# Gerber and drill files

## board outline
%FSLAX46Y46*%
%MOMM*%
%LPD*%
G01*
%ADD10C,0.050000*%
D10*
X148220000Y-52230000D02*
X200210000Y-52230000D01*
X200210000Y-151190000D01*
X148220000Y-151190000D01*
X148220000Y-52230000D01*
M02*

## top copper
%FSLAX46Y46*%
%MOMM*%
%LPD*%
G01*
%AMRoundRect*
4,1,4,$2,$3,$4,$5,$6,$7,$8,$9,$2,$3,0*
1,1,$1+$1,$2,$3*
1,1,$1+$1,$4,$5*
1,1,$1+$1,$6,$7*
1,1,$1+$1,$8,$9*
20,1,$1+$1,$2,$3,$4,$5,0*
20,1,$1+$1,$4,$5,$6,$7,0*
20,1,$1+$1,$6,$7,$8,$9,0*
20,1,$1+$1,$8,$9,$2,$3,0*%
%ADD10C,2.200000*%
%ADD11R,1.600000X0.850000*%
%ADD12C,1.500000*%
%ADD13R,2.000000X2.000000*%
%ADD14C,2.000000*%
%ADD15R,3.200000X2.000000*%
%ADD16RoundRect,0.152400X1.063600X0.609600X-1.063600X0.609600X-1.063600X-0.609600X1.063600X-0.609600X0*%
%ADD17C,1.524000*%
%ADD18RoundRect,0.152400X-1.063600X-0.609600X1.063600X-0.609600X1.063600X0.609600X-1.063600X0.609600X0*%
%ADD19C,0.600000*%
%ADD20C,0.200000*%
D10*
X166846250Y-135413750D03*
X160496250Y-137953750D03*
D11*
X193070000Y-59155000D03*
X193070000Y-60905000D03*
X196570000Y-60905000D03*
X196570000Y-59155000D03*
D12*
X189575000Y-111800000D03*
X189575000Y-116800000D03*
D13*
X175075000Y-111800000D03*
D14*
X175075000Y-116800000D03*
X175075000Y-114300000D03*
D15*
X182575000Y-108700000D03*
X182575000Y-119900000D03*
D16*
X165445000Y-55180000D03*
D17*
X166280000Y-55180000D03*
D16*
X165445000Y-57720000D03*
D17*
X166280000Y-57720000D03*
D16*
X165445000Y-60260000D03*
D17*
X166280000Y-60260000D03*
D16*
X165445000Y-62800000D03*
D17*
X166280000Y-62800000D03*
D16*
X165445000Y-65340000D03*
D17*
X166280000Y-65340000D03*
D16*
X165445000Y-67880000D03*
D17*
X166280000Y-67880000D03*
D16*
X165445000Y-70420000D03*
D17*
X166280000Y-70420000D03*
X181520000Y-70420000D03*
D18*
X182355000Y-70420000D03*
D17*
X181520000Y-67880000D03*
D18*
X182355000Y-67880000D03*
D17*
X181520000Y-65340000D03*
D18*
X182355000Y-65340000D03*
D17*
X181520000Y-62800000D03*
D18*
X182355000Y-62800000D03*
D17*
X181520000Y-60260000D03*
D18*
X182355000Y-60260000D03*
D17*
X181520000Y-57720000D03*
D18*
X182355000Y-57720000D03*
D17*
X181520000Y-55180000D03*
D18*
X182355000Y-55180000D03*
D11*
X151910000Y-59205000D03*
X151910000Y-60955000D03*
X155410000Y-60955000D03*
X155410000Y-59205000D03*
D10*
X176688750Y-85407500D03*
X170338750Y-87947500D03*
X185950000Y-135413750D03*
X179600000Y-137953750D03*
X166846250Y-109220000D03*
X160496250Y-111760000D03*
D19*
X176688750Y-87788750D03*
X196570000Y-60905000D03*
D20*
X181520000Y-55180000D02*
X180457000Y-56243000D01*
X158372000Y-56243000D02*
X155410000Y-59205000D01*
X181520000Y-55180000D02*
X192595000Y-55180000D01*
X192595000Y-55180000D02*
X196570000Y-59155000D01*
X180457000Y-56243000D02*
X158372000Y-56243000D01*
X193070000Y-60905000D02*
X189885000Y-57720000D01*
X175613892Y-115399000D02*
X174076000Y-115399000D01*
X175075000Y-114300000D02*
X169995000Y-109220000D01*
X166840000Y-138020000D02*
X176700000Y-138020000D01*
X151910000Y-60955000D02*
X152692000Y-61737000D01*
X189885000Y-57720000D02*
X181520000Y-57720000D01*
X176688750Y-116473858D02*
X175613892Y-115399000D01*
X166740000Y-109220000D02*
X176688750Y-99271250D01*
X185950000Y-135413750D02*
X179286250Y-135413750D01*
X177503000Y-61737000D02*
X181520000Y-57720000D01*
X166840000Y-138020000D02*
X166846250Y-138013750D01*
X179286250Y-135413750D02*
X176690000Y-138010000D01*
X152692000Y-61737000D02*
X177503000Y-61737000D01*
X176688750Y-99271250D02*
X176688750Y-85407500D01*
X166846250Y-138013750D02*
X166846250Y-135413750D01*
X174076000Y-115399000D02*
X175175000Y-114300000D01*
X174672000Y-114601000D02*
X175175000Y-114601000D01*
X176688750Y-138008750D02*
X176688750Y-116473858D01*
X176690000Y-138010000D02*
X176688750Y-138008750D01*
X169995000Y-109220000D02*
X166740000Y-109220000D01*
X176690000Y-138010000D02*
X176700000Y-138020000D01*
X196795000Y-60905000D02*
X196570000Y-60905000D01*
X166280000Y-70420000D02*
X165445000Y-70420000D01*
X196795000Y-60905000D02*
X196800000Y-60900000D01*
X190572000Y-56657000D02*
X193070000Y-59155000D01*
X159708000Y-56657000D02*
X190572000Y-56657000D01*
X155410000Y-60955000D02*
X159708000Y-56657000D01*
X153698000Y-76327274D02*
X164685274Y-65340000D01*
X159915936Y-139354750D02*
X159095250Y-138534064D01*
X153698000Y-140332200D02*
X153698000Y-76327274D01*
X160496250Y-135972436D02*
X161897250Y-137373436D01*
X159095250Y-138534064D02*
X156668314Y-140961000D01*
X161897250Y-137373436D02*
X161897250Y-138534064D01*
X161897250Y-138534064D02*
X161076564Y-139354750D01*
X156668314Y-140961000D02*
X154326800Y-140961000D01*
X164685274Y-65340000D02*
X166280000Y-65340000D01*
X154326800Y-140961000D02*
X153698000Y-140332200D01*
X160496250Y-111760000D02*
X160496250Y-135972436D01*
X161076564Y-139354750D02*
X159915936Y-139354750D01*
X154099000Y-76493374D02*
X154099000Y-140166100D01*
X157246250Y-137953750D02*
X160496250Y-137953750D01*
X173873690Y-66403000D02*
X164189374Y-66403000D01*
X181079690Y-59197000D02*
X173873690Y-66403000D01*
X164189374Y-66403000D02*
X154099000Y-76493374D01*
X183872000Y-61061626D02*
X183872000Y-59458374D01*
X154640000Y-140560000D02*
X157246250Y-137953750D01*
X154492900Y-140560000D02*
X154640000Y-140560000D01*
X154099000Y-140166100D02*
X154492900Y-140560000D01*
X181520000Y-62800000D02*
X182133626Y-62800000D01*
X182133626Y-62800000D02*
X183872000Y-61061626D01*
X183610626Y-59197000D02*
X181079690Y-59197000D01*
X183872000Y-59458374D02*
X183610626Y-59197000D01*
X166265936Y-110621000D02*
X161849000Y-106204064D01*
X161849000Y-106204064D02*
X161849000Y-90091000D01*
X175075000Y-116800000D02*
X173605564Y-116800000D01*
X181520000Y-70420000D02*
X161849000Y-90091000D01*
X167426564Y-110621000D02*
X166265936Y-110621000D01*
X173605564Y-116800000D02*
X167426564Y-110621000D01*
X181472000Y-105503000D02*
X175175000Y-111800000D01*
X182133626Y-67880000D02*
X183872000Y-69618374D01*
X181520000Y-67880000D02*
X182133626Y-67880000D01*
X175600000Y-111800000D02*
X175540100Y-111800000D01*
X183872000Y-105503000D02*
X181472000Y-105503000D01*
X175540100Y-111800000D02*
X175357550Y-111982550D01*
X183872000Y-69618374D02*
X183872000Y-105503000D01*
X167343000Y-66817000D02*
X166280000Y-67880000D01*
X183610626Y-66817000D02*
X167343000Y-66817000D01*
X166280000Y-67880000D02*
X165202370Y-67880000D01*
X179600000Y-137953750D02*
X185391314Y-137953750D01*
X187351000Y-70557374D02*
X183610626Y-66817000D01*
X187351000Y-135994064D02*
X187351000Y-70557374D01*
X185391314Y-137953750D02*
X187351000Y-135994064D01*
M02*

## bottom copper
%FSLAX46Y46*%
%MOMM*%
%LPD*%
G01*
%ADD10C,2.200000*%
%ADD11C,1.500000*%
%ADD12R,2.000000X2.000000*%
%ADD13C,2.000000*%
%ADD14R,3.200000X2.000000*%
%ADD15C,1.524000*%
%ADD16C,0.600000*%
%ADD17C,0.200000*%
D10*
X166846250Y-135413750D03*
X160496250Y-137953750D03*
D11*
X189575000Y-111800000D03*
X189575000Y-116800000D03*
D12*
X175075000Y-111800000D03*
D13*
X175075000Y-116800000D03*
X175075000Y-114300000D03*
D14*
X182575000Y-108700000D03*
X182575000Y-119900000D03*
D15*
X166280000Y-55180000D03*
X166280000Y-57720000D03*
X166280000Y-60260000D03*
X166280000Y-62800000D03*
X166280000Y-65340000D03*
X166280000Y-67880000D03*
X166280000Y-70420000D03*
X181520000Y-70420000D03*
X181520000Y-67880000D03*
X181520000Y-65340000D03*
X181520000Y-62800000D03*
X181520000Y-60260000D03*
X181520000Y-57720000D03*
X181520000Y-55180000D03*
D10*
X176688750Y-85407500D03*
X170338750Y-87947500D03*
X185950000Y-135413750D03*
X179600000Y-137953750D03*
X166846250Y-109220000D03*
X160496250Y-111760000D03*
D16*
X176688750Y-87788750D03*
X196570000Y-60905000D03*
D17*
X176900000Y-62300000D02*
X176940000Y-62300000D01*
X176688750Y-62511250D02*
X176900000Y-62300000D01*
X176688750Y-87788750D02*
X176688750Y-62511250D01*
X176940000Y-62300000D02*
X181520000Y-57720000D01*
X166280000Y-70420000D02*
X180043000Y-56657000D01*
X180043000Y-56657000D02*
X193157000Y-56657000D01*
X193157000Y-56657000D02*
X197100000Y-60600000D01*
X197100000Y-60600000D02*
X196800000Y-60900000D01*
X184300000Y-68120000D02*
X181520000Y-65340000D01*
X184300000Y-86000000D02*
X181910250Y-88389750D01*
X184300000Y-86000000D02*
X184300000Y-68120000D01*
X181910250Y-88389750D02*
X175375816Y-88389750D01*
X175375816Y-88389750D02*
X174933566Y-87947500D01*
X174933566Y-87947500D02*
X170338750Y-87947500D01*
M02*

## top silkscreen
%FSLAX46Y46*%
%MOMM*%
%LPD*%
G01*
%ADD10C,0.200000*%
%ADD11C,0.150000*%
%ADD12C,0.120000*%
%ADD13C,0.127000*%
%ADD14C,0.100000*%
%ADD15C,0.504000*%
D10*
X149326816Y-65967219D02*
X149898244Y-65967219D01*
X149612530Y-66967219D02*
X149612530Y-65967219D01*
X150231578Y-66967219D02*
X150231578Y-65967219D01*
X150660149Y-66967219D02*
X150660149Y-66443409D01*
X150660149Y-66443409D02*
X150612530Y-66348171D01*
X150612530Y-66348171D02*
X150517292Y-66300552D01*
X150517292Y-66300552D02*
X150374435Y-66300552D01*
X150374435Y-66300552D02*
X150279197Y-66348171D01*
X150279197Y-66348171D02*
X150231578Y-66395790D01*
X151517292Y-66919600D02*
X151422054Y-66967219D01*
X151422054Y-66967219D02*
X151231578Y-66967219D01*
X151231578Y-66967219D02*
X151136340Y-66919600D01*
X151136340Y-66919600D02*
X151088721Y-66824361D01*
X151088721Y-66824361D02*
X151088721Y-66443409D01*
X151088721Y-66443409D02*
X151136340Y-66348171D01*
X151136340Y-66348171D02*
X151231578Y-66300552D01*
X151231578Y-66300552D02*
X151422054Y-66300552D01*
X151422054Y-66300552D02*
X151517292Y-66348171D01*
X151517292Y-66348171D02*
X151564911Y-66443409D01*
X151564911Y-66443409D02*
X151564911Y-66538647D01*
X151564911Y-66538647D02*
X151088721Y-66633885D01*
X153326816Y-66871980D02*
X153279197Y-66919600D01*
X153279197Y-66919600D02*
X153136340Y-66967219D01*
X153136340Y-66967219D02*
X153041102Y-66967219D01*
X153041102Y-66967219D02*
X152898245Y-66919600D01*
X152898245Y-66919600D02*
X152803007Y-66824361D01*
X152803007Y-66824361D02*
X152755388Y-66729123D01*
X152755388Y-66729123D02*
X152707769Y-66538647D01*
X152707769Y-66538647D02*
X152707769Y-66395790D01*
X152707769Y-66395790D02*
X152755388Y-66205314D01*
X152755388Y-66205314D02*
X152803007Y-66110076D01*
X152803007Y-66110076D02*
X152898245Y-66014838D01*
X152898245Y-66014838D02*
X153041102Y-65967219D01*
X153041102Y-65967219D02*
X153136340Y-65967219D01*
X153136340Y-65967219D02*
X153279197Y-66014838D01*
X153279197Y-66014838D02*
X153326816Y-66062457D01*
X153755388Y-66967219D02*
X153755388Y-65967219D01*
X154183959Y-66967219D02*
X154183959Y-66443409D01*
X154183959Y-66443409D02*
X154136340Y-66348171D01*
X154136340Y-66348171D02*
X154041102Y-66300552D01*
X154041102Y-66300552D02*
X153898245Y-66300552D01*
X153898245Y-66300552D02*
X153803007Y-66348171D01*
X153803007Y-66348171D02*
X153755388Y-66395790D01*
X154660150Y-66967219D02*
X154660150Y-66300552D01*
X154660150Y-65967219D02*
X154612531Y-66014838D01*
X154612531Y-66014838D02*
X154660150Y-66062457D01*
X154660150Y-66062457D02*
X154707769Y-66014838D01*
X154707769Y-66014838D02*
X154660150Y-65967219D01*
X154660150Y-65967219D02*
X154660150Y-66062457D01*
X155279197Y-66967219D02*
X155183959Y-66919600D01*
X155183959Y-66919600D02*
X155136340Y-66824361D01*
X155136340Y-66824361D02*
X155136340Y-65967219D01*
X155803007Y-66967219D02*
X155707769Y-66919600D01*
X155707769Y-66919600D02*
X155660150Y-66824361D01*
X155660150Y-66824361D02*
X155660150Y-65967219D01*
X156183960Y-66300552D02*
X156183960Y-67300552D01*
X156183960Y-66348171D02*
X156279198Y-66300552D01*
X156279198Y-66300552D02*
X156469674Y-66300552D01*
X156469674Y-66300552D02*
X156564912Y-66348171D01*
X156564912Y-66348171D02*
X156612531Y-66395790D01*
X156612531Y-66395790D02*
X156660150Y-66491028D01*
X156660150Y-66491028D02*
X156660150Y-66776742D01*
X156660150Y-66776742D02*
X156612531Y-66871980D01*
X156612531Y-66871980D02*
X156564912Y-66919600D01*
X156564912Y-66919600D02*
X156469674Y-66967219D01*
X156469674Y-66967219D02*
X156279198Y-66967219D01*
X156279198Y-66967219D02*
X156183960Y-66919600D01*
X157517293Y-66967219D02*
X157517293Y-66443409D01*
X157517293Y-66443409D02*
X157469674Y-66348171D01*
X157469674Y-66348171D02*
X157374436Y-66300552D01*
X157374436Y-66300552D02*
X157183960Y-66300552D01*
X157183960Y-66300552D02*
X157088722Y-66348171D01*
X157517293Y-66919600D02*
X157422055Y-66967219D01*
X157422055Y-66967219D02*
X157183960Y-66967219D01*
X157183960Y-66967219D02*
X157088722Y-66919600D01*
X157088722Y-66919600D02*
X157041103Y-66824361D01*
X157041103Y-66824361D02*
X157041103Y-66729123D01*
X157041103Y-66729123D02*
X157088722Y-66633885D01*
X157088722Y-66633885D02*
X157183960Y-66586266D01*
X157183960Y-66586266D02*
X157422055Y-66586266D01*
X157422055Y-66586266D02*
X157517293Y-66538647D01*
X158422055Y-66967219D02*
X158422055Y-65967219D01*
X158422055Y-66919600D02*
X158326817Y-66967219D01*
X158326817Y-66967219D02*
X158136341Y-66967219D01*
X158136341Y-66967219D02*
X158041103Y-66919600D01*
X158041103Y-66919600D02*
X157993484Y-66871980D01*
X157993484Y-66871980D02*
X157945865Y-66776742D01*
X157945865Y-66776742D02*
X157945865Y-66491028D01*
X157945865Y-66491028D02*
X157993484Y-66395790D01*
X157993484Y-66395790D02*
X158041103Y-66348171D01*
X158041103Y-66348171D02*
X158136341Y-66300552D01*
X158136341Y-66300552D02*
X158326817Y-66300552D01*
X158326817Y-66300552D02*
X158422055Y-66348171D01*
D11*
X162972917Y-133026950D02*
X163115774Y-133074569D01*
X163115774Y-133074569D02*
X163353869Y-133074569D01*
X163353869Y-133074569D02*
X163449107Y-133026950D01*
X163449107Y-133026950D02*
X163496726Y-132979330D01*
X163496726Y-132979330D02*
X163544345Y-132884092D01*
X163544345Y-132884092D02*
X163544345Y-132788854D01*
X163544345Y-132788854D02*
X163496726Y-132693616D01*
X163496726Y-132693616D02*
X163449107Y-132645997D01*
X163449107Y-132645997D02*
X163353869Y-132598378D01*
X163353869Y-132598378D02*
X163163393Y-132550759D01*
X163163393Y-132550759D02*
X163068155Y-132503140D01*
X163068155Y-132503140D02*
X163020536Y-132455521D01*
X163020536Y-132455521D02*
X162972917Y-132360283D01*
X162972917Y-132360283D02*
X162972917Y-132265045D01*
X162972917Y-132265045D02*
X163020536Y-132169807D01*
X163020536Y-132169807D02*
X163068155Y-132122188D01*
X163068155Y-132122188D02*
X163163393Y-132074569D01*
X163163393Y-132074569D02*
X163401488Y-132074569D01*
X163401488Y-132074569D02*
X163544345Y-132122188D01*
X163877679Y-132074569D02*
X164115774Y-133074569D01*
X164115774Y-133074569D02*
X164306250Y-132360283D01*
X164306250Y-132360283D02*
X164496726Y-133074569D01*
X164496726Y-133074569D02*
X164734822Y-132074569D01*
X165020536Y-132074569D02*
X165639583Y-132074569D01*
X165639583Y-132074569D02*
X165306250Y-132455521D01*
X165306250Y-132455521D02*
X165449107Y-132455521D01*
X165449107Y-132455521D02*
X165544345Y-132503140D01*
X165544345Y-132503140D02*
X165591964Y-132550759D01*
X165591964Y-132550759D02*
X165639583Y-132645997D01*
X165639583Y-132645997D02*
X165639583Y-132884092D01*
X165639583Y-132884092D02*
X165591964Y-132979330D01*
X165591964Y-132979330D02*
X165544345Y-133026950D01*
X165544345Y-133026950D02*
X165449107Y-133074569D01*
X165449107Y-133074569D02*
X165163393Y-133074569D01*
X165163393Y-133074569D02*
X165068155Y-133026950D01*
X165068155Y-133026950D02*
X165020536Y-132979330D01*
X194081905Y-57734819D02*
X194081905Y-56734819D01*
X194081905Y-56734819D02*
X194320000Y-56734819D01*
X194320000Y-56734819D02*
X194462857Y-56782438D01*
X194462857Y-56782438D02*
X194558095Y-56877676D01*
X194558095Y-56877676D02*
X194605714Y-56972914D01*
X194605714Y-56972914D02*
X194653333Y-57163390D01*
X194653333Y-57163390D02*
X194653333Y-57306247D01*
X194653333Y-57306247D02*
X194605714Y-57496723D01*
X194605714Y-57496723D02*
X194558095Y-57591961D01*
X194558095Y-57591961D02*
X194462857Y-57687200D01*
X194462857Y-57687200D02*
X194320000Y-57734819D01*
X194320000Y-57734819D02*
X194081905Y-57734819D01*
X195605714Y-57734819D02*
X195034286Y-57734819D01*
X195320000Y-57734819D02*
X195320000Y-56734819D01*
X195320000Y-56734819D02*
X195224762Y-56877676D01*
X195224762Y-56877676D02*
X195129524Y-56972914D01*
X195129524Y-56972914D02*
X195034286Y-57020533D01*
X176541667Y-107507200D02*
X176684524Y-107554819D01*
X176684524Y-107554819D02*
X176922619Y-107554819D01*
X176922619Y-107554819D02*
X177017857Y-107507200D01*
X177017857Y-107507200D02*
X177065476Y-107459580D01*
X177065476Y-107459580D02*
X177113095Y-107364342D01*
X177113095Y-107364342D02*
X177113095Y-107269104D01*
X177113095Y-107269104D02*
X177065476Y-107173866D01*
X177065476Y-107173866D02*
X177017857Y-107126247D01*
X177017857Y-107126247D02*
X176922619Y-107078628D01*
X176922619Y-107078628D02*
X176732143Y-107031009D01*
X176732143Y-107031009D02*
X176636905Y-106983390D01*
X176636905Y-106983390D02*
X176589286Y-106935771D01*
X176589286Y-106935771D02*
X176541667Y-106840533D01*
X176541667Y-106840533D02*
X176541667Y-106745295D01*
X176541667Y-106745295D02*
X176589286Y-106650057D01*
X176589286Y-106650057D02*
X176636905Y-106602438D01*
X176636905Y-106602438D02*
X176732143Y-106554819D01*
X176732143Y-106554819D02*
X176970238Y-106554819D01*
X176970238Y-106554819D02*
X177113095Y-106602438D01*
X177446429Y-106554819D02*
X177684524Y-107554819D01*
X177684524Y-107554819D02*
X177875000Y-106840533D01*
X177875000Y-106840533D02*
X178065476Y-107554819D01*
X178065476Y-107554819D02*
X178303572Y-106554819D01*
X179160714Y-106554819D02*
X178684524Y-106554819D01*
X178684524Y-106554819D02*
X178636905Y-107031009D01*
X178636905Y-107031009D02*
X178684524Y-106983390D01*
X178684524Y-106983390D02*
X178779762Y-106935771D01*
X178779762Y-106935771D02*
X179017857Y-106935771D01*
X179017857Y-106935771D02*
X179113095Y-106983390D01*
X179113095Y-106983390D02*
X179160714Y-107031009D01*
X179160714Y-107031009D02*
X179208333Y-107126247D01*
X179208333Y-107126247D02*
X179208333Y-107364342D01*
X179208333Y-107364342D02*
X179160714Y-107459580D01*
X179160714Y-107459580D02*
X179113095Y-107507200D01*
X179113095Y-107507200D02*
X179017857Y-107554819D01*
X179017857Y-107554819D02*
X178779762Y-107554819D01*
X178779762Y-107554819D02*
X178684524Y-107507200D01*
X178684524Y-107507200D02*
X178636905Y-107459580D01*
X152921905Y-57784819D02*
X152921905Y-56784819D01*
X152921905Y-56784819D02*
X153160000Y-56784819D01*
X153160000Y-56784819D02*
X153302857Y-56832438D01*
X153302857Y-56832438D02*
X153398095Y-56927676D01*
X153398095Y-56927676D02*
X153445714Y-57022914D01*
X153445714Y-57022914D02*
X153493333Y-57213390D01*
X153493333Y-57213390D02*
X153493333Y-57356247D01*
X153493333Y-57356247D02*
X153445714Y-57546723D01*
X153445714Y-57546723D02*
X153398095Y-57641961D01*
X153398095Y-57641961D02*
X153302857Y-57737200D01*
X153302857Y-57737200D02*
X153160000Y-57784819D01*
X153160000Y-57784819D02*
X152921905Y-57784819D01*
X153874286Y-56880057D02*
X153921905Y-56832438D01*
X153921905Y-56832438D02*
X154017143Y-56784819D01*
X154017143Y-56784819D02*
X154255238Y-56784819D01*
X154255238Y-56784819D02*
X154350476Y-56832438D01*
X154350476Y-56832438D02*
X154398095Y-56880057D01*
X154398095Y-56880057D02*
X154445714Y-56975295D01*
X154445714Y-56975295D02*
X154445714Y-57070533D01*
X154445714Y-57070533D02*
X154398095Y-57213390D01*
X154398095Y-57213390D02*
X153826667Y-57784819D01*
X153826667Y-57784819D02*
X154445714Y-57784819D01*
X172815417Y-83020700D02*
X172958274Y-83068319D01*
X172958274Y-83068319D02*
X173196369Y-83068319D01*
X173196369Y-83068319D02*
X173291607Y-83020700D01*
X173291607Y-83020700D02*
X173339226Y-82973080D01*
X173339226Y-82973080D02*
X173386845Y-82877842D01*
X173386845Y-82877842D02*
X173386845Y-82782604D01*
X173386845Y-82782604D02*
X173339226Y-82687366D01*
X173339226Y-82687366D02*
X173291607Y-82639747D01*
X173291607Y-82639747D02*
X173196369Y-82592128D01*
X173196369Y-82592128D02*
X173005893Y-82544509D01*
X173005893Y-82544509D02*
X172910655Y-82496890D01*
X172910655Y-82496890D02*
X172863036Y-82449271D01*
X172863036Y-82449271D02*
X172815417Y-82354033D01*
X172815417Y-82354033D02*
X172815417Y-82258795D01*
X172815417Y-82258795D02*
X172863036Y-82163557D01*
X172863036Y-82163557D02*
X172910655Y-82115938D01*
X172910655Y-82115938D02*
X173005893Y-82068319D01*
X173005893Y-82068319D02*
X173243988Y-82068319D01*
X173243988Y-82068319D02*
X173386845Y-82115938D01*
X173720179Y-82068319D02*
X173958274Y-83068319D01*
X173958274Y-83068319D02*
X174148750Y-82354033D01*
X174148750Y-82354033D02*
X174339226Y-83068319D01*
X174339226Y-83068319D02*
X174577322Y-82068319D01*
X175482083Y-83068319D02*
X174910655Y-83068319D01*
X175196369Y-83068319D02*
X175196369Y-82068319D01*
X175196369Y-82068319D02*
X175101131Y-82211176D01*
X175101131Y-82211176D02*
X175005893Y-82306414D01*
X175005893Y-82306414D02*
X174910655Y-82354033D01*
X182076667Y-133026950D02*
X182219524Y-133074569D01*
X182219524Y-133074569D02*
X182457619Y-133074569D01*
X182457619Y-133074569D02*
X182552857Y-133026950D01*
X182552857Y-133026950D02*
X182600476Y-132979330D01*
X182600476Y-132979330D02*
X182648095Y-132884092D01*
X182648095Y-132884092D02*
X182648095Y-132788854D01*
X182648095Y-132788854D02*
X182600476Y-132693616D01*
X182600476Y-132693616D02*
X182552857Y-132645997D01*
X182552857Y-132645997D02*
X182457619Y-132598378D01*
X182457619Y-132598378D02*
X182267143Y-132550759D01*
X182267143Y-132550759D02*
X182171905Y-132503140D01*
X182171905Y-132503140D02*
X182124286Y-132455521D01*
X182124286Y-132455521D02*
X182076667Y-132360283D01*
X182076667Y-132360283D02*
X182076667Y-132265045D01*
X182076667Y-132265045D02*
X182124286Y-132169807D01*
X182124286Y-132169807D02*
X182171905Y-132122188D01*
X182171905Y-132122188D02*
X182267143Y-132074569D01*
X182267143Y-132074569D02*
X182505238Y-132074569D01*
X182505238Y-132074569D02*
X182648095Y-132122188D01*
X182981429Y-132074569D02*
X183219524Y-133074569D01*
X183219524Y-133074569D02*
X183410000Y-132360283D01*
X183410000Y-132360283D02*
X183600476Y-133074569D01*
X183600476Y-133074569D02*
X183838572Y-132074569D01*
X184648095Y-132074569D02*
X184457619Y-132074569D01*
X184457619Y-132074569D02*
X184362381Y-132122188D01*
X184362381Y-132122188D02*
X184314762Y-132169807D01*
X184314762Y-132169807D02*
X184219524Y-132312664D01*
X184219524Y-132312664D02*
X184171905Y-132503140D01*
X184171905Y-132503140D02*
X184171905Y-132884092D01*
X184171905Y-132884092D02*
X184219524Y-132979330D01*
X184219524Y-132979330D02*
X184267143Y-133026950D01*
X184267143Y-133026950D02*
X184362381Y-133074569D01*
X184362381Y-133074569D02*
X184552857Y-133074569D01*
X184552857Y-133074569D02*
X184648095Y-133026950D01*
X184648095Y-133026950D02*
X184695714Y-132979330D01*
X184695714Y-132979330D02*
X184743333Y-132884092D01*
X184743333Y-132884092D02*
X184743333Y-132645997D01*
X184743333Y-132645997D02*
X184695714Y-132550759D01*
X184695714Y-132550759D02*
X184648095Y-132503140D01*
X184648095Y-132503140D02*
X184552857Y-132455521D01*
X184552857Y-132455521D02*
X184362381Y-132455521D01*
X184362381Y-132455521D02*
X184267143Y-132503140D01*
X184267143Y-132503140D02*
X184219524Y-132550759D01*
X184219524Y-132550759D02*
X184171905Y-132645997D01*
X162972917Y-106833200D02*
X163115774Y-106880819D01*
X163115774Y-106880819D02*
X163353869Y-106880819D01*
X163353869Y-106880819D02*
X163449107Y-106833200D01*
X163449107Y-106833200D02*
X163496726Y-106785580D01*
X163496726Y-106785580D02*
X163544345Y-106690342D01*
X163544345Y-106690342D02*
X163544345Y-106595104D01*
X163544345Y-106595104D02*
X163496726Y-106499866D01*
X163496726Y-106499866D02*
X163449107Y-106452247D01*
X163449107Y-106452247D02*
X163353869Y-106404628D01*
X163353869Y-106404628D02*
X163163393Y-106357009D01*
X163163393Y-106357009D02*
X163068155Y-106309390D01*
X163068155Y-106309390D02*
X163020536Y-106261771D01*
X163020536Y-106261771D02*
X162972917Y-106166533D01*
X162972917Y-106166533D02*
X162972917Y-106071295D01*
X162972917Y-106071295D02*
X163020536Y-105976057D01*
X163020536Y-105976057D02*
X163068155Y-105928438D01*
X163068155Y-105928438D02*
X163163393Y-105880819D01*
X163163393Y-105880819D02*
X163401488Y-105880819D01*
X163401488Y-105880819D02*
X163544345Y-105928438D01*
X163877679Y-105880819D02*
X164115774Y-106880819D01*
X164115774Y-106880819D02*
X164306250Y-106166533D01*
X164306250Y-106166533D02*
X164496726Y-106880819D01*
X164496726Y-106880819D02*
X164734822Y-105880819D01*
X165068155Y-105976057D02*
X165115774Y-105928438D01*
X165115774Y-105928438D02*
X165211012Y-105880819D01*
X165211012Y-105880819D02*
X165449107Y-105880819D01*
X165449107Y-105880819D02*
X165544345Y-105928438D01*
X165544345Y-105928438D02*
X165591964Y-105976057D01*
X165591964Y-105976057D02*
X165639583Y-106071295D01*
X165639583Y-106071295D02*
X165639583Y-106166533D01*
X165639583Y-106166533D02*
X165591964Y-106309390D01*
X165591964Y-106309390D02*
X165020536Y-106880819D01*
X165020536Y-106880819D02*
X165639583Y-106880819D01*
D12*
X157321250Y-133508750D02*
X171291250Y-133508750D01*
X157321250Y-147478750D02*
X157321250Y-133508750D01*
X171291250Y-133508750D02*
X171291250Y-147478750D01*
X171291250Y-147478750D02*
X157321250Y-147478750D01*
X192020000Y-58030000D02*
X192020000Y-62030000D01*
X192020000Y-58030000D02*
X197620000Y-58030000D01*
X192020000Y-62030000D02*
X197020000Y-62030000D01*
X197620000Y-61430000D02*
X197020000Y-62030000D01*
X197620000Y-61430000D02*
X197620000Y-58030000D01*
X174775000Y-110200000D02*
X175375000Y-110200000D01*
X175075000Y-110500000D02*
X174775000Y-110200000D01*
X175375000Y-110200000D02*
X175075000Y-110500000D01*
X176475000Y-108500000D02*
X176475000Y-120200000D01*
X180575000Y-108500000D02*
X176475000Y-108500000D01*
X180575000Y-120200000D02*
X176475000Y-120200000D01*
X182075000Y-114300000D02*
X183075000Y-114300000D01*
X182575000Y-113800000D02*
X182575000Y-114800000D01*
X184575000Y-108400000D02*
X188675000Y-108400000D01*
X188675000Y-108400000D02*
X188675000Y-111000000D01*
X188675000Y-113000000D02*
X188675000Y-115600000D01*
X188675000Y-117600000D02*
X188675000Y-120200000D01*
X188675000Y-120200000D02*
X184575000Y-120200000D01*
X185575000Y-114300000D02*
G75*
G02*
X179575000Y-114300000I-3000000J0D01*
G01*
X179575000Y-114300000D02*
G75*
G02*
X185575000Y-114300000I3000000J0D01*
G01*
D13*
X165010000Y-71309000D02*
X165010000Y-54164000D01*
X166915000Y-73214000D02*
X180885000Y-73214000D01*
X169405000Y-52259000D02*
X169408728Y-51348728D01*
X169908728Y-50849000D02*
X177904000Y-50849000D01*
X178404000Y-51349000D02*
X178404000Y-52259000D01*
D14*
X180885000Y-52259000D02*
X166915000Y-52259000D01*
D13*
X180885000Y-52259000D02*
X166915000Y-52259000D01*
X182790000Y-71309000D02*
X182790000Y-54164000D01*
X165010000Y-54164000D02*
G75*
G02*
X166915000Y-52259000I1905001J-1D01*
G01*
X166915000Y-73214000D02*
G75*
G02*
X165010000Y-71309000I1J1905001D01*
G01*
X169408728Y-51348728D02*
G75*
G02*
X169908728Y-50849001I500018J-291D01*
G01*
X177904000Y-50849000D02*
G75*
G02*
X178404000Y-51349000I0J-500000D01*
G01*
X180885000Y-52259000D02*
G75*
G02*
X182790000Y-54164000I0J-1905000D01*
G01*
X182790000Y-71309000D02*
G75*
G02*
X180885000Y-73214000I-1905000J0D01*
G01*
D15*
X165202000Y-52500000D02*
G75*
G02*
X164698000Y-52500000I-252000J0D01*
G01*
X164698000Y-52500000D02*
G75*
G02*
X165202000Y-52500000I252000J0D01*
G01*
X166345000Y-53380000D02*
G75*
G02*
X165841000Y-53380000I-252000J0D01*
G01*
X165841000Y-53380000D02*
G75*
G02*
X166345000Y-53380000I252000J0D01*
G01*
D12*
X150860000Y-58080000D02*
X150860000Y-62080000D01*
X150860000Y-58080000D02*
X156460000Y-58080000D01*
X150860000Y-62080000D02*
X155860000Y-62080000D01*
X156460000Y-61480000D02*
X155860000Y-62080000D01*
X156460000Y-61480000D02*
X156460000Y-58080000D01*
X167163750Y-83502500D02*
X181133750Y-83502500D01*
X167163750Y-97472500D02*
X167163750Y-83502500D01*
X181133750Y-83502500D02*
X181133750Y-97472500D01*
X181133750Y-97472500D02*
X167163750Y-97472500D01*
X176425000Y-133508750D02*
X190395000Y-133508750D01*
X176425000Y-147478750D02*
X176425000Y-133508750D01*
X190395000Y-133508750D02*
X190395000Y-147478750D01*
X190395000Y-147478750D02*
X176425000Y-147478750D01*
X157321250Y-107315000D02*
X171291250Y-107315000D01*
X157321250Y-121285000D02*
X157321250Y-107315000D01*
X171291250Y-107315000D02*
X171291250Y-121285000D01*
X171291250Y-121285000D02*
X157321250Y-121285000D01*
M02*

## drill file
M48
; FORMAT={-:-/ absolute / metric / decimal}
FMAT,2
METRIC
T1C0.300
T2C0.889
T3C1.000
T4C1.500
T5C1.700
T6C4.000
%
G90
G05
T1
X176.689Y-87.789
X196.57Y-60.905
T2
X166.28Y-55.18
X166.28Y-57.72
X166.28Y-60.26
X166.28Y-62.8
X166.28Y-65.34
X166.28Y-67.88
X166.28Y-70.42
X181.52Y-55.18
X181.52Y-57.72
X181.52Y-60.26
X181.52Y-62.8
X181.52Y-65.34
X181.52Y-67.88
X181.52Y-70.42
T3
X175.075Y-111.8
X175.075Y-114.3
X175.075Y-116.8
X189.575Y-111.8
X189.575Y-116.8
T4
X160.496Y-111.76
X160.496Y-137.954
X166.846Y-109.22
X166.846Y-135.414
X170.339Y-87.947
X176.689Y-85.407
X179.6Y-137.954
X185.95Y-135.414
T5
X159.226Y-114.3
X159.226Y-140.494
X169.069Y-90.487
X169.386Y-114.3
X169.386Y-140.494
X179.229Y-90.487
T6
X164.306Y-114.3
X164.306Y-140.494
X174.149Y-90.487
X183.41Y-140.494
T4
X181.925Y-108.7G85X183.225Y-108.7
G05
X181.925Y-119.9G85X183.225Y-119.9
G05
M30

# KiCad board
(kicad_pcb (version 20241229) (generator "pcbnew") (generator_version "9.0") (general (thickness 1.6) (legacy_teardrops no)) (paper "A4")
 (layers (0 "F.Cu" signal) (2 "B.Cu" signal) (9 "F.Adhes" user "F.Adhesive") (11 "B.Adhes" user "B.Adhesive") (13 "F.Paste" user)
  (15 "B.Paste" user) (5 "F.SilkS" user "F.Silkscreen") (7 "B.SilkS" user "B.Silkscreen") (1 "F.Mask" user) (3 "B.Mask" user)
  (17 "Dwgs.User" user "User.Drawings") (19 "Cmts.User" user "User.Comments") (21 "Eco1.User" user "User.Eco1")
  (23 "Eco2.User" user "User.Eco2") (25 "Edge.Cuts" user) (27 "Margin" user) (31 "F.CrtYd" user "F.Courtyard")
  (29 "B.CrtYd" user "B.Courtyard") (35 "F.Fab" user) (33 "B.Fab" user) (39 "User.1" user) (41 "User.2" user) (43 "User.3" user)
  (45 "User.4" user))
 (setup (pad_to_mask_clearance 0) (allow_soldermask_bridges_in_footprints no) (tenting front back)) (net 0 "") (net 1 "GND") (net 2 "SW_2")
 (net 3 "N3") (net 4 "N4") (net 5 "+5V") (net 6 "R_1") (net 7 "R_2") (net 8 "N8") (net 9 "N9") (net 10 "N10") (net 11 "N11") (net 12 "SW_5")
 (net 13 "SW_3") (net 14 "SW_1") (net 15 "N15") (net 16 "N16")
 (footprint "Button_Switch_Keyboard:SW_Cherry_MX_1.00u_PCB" (layer "F.Cu") (at 166.84625 135.41375)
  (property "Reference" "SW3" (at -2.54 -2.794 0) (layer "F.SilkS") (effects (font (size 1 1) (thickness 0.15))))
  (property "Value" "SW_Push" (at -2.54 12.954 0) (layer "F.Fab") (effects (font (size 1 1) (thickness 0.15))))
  (fp_line (start -9.525 -1.905) (end 4.445 -1.905) (stroke (width 0.12) (type solid)) (layer "F.SilkS"))
  (fp_line (start -9.525 12.065) (end -9.525 -1.905) (stroke (width 0.12) (type solid)) (layer "F.SilkS"))
  (fp_line (start 4.445 -1.905) (end 4.445 12.065) (stroke (width 0.12) (type solid)) (layer "F.SilkS"))
  (fp_line (start 4.445 12.065) (end -9.525 12.065) (stroke (width 0.12) (type solid)) (layer "F.SilkS"))
  (pad "" np_thru_hole circle (at -7.62 5.08) (size 1.7 1.7) (drill 1.7) (layers "*.Cu" "*.Mask"))
  (pad "" np_thru_hole circle (at -2.54 5.08) (size 4 4) (drill 4) (layers "*.Cu" "*.Mask"))
  (pad "" np_thru_hole circle (at 2.54 5.08) (size 1.7 1.7) (drill 1.7) (layers "*.Cu" "*.Mask"))
  (pad "1" thru_hole circle (at 0 0) (size 2.2 2.2) (drill 1.5) (layers "*.Cu" "*.Mask") (remove_unused_layers no) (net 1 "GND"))
  (pad "2" thru_hole circle (at -6.35 2.54) (size 2.2 2.2) (drill 1.5) (layers "*.Cu" "*.Mask") (remove_unused_layers no) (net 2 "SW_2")))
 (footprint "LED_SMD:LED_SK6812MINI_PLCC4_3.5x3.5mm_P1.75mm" (layer "F.Cu") (at 194.82 60.03)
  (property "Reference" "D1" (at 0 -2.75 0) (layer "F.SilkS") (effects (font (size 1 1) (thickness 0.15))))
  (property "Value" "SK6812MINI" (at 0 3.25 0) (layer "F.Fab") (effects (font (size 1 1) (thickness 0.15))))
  (fp_line (start -2.8 -2) (end -2.8 2) (stroke (width 0.12) (type default)) (layer "F.SilkS"))
  (fp_line (start -2.8 -2) (end 2.8 -2) (stroke (width 0.12) (type solid)) (layer "F.SilkS"))
  (fp_line (start -2.8 2) (end 2.2 2) (stroke (width 0.12) (type solid)) (layer "F.SilkS"))
  (fp_line (start 2.8 1.4) (end 2.2 2) (stroke (width 0.12) (type default)) (layer "F.SilkS"))
  (fp_line (start 2.8 1.4) (end 2.8 -2) (stroke (width 0.12) (type solid)) (layer "F.SilkS"))
  (pad "1" smd rect (at -1.75 -0.875) (size 1.6 0.85) (layers "F.Cu" "F.Mask" "F.Paste") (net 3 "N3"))
  (pad "2" smd rect (at -1.75 0.875) (size 1.6 0.85) (layers "F.Cu" "F.Mask" "F.Paste") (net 1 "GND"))
  (pad "3" smd rect (at 1.75 0.875) (size 1.6 0.85) (layers "F.Cu" "F.Mask" "F.Paste") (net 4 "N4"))
  (pad "4" smd rect (at 1.75 -0.875) (size 1.6 0.85) (layers "F.Cu" "F.Mask" "F.Paste") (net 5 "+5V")))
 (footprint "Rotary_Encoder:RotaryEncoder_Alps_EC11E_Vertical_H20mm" (layer "F.Cu") (at 175.075 111.8)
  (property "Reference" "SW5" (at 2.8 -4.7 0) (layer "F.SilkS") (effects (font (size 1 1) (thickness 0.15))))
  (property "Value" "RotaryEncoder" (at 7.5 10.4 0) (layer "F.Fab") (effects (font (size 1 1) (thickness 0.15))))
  (fp_line (start -0.3 -1.6) (end 0.3 -1.6) (stroke (width 0.12) (type solid)) (layer "F.SilkS"))
  (fp_line (start 0 -1.3) (end -0.3 -1.6) (stroke (width 0.12) (type solid)) (layer "F.SilkS"))
  (fp_line (start 0.3 -1.6) (end 0 -1.3) (stroke (width 0.12) (type solid)) (layer "F.SilkS"))
  (fp_line (start 1.4 -3.3) (end 1.4 8.4) (stroke (width 0.12) (type solid)) (layer "F.SilkS"))
  (fp_line (start 5.5 -3.3) (end 1.4 -3.3) (stroke (width 0.12) (type solid)) (layer "F.SilkS"))
  (fp_line (start 5.5 8.4) (end 1.4 8.4) (stroke (width 0.12) (type solid)) (layer "F.SilkS"))
  (fp_line (start 7 2.5) (end 8 2.5) (stroke (width 0.12) (type solid)) (layer "F.SilkS"))
  (fp_line (start 7.5 2) (end 7.5 3) (stroke (width 0.12) (type solid)) (layer "F.SilkS"))
  (fp_line (start 9.5 -3.4) (end 13.6 -3.4) (stroke (width 0.12) (type solid)) (layer "F.SilkS"))
  (fp_line (start 13.6 -3.4) (end 13.6 -0.8) (stroke (width 0.12) (type solid)) (layer "F.SilkS"))
  (fp_line (start 13.6 1.2) (end 13.6 3.8) (stroke (width 0.12) (type solid)) (layer "F.SilkS"))
  (fp_line (start 13.6 5.8) (end 13.6 8.4) (stroke (width 0.12) (type solid)) (layer "F.SilkS"))
  (fp_line (start 13.6 8.4) (end 9.5 8.4) (stroke (width 0.12) (type solid)) (layer "F.SilkS"))
  (fp_circle (center 7.5 2.5) (end 10.5 2.5) (stroke (width 0.12) (type solid)) (fill no) (layer "F.SilkS"))
  (pad "" thru_hole circle (at 14.5 0) (size 1.5 1.5) (drill 1) (layers "*.Cu" "*.Mask") (remove_unused_layers no))
  (pad "" thru_hole circle (at 14.5 5) (size 1.5 1.5) (drill 1) (layers "*.Cu" "*.Mask") (remove_unused_layers no))
  (pad "A" thru_hole rect (at 0 0) (size 2 2) (drill 1) (layers "*.Cu" "*.Mask") (remove_unused_layers no) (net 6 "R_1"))
  (pad "B" thru_hole circle (at 0 5) (size 2 2) (drill 1) (layers "*.Cu" "*.Mask") (remove_unused_layers no) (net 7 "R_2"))
  (pad "C" thru_hole circle (at 0 2.5) (size 2 2) (drill 1) (layers "*.Cu" "*.Mask") (remove_unused_layers no) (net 1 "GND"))
  (pad "MP" thru_hole rect (at 7.5 -3.1) (size 3.2 2) (drill oval 2.8 1.5) (layers "*.Cu" "*.Mask") (remove_unused_layers no))
  (pad "MP" thru_hole rect (at 7.5 8.1) (size 3.2 2) (drill oval 2.8 1.5) (layers "*.Cu" "*.Mask") (remove_unused_layers no)))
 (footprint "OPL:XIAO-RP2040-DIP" (layer "F.Cu") (at 173.9 62.8)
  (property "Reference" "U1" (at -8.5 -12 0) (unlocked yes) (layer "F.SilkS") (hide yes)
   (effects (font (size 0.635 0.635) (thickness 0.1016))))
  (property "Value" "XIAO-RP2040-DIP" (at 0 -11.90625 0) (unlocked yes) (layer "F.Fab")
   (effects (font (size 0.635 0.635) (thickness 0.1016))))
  (fp_line (start -8.89 8.509) (end -8.89 -8.636) (stroke (width 0.127) (type solid)) (layer "F.SilkS"))
  (fp_line (start -6.985 10.414) (end 6.985 10.414) (stroke (width 0.127) (type solid)) (layer "F.SilkS"))
  (fp_line (start -4.495 -10.541) (end -4.491272 -11.451272) (stroke (width 0.127) (type solid)) (layer "F.SilkS"))
  (fp_line (start -3.991272 -11.951) (end 4.004 -11.951) (stroke (width 0.127) (type solid)) (layer "F.SilkS"))
  (fp_line (start 4.504 -11.451) (end 4.504 -10.541) (stroke (width 0.127) (type solid)) (layer "F.SilkS"))
  (fp_line (start 6.985 -10.541) (end -6.985 -10.541) (stroke (width 0.1) (type solid)) (layer "F.SilkS"))
  (fp_line (start 6.985 -10.541) (end -6.985 -10.541) (stroke (width 0.127) (type solid)) (layer "F.SilkS"))
  (fp_line (start 8.89 8.509) (end 8.89 -8.636) (stroke (width 0.127) (type solid)) (layer "F.SilkS"))
  (fp_arc (start -8.89 -8.636) (mid -8.332038 -9.983038) (end -6.985 -10.541) (stroke (width 0.127) (type solid)) (layer "F.SilkS"))
  (fp_arc (start -6.985 10.414) (mid -8.332038 9.856038) (end -8.89 8.509) (stroke (width 0.127) (type solid)) (layer "F.SilkS"))
  (fp_arc (start -4.491272 -11.451272) (mid -4.344728 -11.80464) (end -3.991272 -11.951) (stroke (width 0.127) (type default))
   (layer "F.SilkS"))
  (fp_arc (start 4.004 -11.951) (mid 4.357553 -11.804553) (end 4.504 -11.451) (stroke (width 0.127) (type default)) (layer "F.SilkS"))
  (fp_arc (start 6.985 -10.541) (mid 8.332038 -9.983038) (end 8.89 -8.636) (stroke (width 0.127) (type solid)) (layer "F.SilkS"))
  (fp_arc (start 8.89 8.509) (mid 8.332038 9.856038) (end 6.985 10.414) (stroke (width 0.127) (type solid)) (layer "F.SilkS"))
  (fp_circle (center -8.95 -10.3) (end -8.95 -10.554) (stroke (width 0.5) (type solid)) (fill yes) (layer "F.SilkS"))
  (fp_circle (center -7.807 -9.42) (end -7.807 -9.674) (stroke (width 0.5) (type solid)) (fill yes) (layer "F.SilkS"))
  (pad "1" smd roundrect (at -8.455 -7.62 180) (size 2.432 1.524) (layers "F.Cu" "F.Mask") (roundrect_rratio 0.1) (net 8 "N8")
   (thermal_bridge_angle 45))
  (pad "1" thru_hole circle (at -7.62 -7.62 180) (size 1.524 1.524) (drill 0.889) (layers "*.Cu" "*.Mask") (remove_unused_layers no)
   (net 8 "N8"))
  (pad "2" smd roundrect (at -8.455 -5.08 180) (size 2.432 1.524) (layers "F.Cu" "F.Mask") (roundrect_rratio 0.1) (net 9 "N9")
   (thermal_bridge_angle 45))
  (pad "2" thru_hole circle (at -7.62 -5.08 180) (size 1.524 1.524) (drill 0.889) (layers "*.Cu" "*.Mask") (remove_unused_layers no)
   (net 9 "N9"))
  (pad "3" smd roundrect (at -8.455 -2.54 180) (size 2.432 1.524) (layers "F.Cu" "F.Mask") (roundrect_rratio 0.1) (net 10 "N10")
   (thermal_bridge_angle 45))
  (pad "3" thru_hole circle (at -7.62 -2.54 180) (size 1.524 1.524) (drill 0.889) (layers "*.Cu" "*.Mask") (remove_unused_layers no)
   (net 10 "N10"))
  (pad "4" smd roundrect (at -8.455 0 180) (size 2.432 1.524) (layers "F.Cu" "F.Mask") (roundrect_rratio 0.1) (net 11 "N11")
   (thermal_bridge_angle 45))
  (pad "4" thru_hole circle (at -7.62 0 180) (size 1.524 1.524) (drill 0.889) (layers "*.Cu" "*.Mask") (remove_unused_layers no)
   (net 11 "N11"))
  (pad "5" smd roundrect (at -8.455 2.54 180) (size 2.432 1.524) (layers "F.Cu" "F.Mask") (roundrect_rratio 0.1) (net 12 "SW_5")
   (thermal_bridge_angle 45))
  (pad "5" thru_hole circle (at -7.62 2.54 180) (size 1.524 1.524) (drill 0.889) (layers "*.Cu" "*.Mask") (remove_unused_layers no)
   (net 12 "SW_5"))
  (pad "6" smd roundrect (at -8.455 5.08 180) (size 2.432 1.524) (layers "F.Cu" "F.Mask") (roundrect_rratio 0.1) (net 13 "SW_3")
   (thermal_bridge_angle 45))
  (pad "6" thru_hole circle (at -7.62 5.08 180) (size 1.524 1.524) (drill 0.889) (layers "*.Cu" "*.Mask") (remove_unused_layers no)
   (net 13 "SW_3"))
  (pad "7" smd roundrect (at -8.455 7.62 180) (size 2.432 1.524) (layers "F.Cu" "F.Mask") (roundrect_rratio 0.1) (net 4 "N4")
   (thermal_bridge_angle 45))
  (pad "7" thru_hole circle (at -7.62 7.62 180) (size 1.524 1.524) (drill 0.889) (layers "*.Cu" "*.Mask") (remove_unused_layers no)
   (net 4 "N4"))
  (pad "8" thru_hole circle (at 7.62 7.62) (size 1.524 1.524) (drill 0.889) (layers "*.Cu" "*.Mask") (remove_unused_layers no) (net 7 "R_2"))
  (pad "8" smd roundrect (at 8.455 7.62) (size 2.432 1.524) (layers "F.Cu" "F.Mask") (roundrect_rratio 0.1) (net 7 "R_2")
   (thermal_bridge_angle 45))
  (pad "9" thru_hole circle (at 7.62 5.08) (size 1.524 1.524) (drill 0.889) (layers "*.Cu" "*.Mask") (remove_unused_layers no) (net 6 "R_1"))
  (pad "9" smd roundrect (at 8.455 5.08) (size 2.432 1.524) (layers "F.Cu" "F.Mask") (roundrect_rratio 0.1) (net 6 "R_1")
   (thermal_bridge_angle 45))
  (pad "10" thru_hole circle (at 7.62 2.54) (size 1.524 1.524) (drill 0.889) (layers "*.Cu" "*.Mask") (remove_unused_layers no)
   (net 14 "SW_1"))
  (pad "10" smd roundrect (at 8.455 2.54) (size 2.432 1.524) (layers "F.Cu" "F.Mask") (roundrect_rratio 0.1) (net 14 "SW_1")
   (thermal_bridge_angle 45))
  (pad "11" thru_hole circle (at 7.62 0) (size 1.524 1.524) (drill 0.889) (layers "*.Cu" "*.Mask") (remove_unused_layers no) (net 2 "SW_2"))
  (pad "11" smd roundrect (at 8.455 0) (size 2.432 1.524) (layers "F.Cu" "F.Mask") (roundrect_rratio 0.1) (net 2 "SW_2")
   (thermal_bridge_angle 45))
  (pad "12" thru_hole circle (at 7.62 -2.54) (size 1.524 1.524) (drill 0.889) (layers "*.Cu" "*.Mask") (remove_unused_layers no)
   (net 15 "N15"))
  (pad "12" smd roundrect (at 8.455 -2.54) (size 2.432 1.524) (layers "F.Cu" "F.Mask") (roundrect_rratio 0.1) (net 15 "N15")
   (thermal_bridge_angle 45))
  (pad "13" thru_hole circle (at 7.62 -5.08) (size 1.524 1.524) (drill 0.889) (layers "*.Cu" "*.Mask") (remove_unused_layers no)
   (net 1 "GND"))
  (pad "13" smd roundrect (at 8.455 -5.08) (size 2.432 1.524) (layers "F.Cu" "F.Mask") (roundrect_rratio 0.1) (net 1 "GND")
   (thermal_bridge_angle 45))
  (pad "14" thru_hole circle (at 7.62 -7.62) (size 1.524 1.524) (drill 0.889) (layers "*.Cu" "*.Mask") (remove_unused_layers no)
   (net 5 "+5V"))
  (pad "14" smd roundrect (at 8.455 -7.62) (size 2.432 1.524) (layers "F.Cu" "F.Mask") (roundrect_rratio 0.1) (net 5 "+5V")
   (thermal_bridge_angle 45)))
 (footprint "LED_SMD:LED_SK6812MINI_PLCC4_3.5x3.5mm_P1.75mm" (layer "F.Cu") (at 153.66 60.08)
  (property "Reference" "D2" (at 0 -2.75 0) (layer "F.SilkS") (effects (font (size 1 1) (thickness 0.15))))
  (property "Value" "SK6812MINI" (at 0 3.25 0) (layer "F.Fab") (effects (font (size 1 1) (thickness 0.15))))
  (fp_line (start -2.8 -2) (end -2.8 2) (stroke (width 0.12) (type default)) (layer "F.SilkS"))
  (fp_line (start -2.8 -2) (end 2.8 -2) (stroke (width 0.12) (type solid)) (layer "F.SilkS"))
  (fp_line (start -2.8 2) (end 2.2 2) (stroke (width 0.12) (type solid)) (layer "F.SilkS"))
  (fp_line (start 2.8 1.4) (end 2.2 2) (stroke (width 0.12) (type default)) (layer "F.SilkS"))
  (fp_line (start 2.8 1.4) (end 2.8 -2) (stroke (width 0.12) (type solid)) (layer "F.SilkS"))
  (pad "1" smd rect (at -1.75 -0.875) (size 1.6 0.85) (layers "F.Cu" "F.Mask" "F.Paste") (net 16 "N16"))
  (pad "2" smd rect (at -1.75 0.875) (size 1.6 0.85) (layers "F.Cu" "F.Mask" "F.Paste") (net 1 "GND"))
  (pad "3" smd rect (at 1.75 0.875) (size 1.6 0.85) (layers "F.Cu" "F.Mask" "F.Paste") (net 3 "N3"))
  (pad "4" smd rect (at 1.75 -0.875) (size 1.6 0.85) (layers "F.Cu" "F.Mask" "F.Paste") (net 5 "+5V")))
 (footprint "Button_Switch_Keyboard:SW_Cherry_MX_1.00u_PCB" (layer "F.Cu") (at 176.68875 85.4075)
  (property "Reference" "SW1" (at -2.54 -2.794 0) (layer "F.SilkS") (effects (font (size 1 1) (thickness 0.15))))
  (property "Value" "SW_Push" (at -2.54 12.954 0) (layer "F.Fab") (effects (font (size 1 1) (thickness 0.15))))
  (fp_line (start -9.525 -1.905) (end 4.445 -1.905) (stroke (width 0.12) (type solid)) (layer "F.SilkS"))
  (fp_line (start -9.525 12.065) (end -9.525 -1.905) (stroke (width 0.12) (type solid)) (layer "F.SilkS"))
  (fp_line (start 4.445 -1.905) (end 4.445 12.065) (stroke (width 0.12) (type solid)) (layer "F.SilkS"))
  (fp_line (start 4.445 12.065) (end -9.525 12.065) (stroke (width 0.12) (type solid)) (layer "F.SilkS"))
  (pad "" np_thru_hole circle (at -7.62 5.08) (size 1.7 1.7) (drill 1.7) (layers "*.Cu" "*.Mask"))
  (pad "" np_thru_hole circle (at -2.54 5.08) (size 4 4) (drill 4) (layers "*.Cu" "*.Mask"))
  (pad "" np_thru_hole circle (at 2.54 5.08) (size 1.7 1.7) (drill 1.7) (layers "*.Cu" "*.Mask"))
  (pad "1" thru_hole circle (at 0 0) (size 2.2 2.2) (drill 1.5) (layers "*.Cu" "*.Mask") (remove_unused_layers no) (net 1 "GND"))
  (pad "2" thru_hole circle (at -6.35 2.54) (size 2.2 2.2) (drill 1.5) (layers "*.Cu" "*.Mask") (remove_unused_layers no) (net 14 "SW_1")))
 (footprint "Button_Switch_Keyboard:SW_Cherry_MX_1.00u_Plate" (layer "F.Cu") (at 185.95 135.41375)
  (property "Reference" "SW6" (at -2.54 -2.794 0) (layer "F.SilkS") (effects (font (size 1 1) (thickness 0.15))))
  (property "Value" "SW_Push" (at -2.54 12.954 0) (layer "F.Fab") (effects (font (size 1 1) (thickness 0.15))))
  (fp_line (start -9.525 -1.905) (end 4.445 -1.905) (stroke (width 0.12) (type solid)) (layer "F.SilkS"))
  (fp_line (start -9.525 12.065) (end -9.525 -1.905) (stroke (width 0.12) (type solid)) (layer "F.SilkS"))
  (fp_line (start 4.445 -1.905) (end 4.445 12.065) (stroke (width 0.12) (type solid)) (layer "F.SilkS"))
  (fp_line (start 4.445 12.065) (end -9.525 12.065) (stroke (width 0.12) (type solid)) (layer "F.SilkS"))
  (pad "" np_thru_hole circle (at -2.54 5.08) (size 4 4) (drill 4) (layers "*.Cu" "*.Mask"))
  (pad "1" thru_hole circle (at 0 0) (size 2.2 2.2) (drill 1.5) (layers "*.Cu" "*.Mask") (remove_unused_layers no) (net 1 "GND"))
  (pad "2" thru_hole circle (at -6.35 2.54) (size 2.2 2.2) (drill 1.5) (layers "*.Cu" "*.Mask") (remove_unused_layers no) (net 13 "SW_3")))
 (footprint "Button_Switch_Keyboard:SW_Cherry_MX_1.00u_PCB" (layer "F.Cu") (at 166.84625 109.22)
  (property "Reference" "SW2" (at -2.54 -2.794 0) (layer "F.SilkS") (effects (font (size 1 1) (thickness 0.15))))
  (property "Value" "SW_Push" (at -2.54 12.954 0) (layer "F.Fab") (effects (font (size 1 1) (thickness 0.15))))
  (fp_line (start -9.525 -1.905) (end 4.445 -1.905) (stroke (width 0.12) (type solid)) (layer "F.SilkS"))
  (fp_line (start -9.525 12.065) (end -9.525 -1.905) (stroke (width 0.12) (type solid)) (layer "F.SilkS"))
  (fp_line (start 4.445 -1.905) (end 4.445 12.065) (stroke (width 0.12) (type solid)) (layer "F.SilkS"))
  (fp_line (start 4.445 12.065) (end -9.525 12.065) (stroke (width 0.12) (type solid)) (layer "F.SilkS"))
  (pad "" np_thru_hole circle (at -7.62 5.08) (size 1.7 1.7) (drill 1.7) (layers "*.Cu" "*.Mask"))
  (pad "" np_thru_hole circle (at -2.54 5.08) (size 4 4) (drill 4) (layers "*.Cu" "*.Mask"))
  (pad "" np_thru_hole circle (at 2.54 5.08) (size 1.7 1.7) (drill 1.7) (layers "*.Cu" "*.Mask"))
  (pad "1" thru_hole circle (at 0 0) (size 2.2 2.2) (drill 1.5) (layers "*.Cu" "*.Mask") (remove_unused_layers no) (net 1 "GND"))
  (pad "2" thru_hole circle (at -6.35 2.54) (size 2.2 2.2) (drill 1.5) (layers "*.Cu" "*.Mask") (remove_unused_layers no) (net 12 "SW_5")))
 (gr_rect (start 148.22 52.23) (end 200.21 151.19) (stroke (width 0.05) (type default)) (fill no) (layer "Edge.Cuts"))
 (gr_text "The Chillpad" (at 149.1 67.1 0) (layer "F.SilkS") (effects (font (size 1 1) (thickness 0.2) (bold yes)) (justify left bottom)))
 (segment (start 181.52 55.18) (end 180.457 56.243) (width 0.2) (layer "F.Cu") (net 5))
 (segment (start 158.372 56.243) (end 155.41 59.205) (width 0.2) (layer "F.Cu") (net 5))
 (segment (start 181.52 55.18) (end 192.595 55.18) (width 0.2) (layer "F.Cu") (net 5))
 (segment (start 192.595 55.18) (end 196.57 59.155) (width 0.2) (layer "F.Cu") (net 5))
 (segment (start 180.457 56.243) (end 158.372 56.243) (width 0.2) (layer "F.Cu") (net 5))
 (segment (start 193.07 60.905) (end 189.885 57.72) (width 0.2) (layer "F.Cu") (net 1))
 (segment (start 175.613892 115.399) (end 174.076 115.399) (width 0.2) (layer "F.Cu") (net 1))
 (segment (start 175.075 114.3) (end 169.995 109.22) (width 0.2) (layer "F.Cu") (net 1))
 (segment (start 166.84 138.02) (end 176.7 138.02) (width 0.2) (layer "F.Cu") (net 1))
 (segment (start 151.91 60.955) (end 152.692 61.737) (width 0.2) (layer "F.Cu") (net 1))
 (segment (start 189.885 57.72) (end 181.52 57.72) (width 0.2) (layer "F.Cu") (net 1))
 (segment (start 176.68875 116.473858) (end 175.613892 115.399) (width 0.2) (layer "F.Cu") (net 1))
 (segment (start 166.74 109.22) (end 176.68875 99.27125) (width 0.2) (layer "F.Cu") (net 1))
 (segment (start 185.95 135.41375) (end 179.28625 135.41375) (width 0.2) (layer "F.Cu") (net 1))
 (segment (start 177.503 61.737) (end 181.52 57.72) (width 0.2) (layer "F.Cu") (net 1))
 (segment (start 166.84 138.02) (end 166.84625 138.01375) (width 0.2) (layer "F.Cu") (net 1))
 (segment (start 179.28625 135.41375) (end 176.69 138.01) (width 0.2) (layer "F.Cu") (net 1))
 (segment (start 152.692 61.737) (end 177.503 61.737) (width 0.2) (layer "F.Cu") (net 1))
 (segment (start 176.68875 99.27125) (end 176.68875 85.4075) (width 0.2) (layer "F.Cu") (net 1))
 (segment (start 166.84625 138.01375) (end 166.84625 135.41375) (width 0.2) (layer "F.Cu") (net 1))
 (segment (start 174.076 115.399) (end 175.175 114.3) (width 0.2) (layer "F.Cu") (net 1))
 (segment (start 174.672 114.601) (end 175.175 114.601) (width 0.2) (layer "F.Cu") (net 1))
 (segment (start 176.68875 138.00875) (end 176.68875 116.473858) (width 0.2) (layer "F.Cu") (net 1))
 (segment (start 176.69 138.01) (end 176.68875 138.00875) (width 0.2) (layer "F.Cu") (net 1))
 (segment (start 169.995 109.22) (end 166.74 109.22) (width 0.2) (layer "F.Cu") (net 1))
 (segment (start 176.69 138.01) (end 176.7 138.02) (width 0.2) (layer "F.Cu") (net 1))
 (via (at 176.68875 87.78875) (size 0.6) (drill 0.3) (layers "F.Cu" "B.Cu") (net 1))
 (segment (start 176.9 62.3) (end 176.94 62.3) (width 0.2) (layer "B.Cu") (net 1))
 (segment (start 176.68875 62.51125) (end 176.9 62.3) (width 0.2) (layer "B.Cu") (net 1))
 (segment (start 176.68875 87.78875) (end 176.68875 62.51125) (width 0.2) (layer "B.Cu") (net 1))
 (segment (start 176.94 62.3) (end 181.52 57.72) (width 0.2) (layer "B.Cu") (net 1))
 (segment (start 196.795 60.905) (end 196.57 60.905) (width 0.2) (layer "F.Cu") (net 4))
 (segment (start 166.28 70.42) (end 165.445 70.42) (width 0.2) (layer "F.Cu") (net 4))
 (segment (start 196.795 60.905) (end 196.8 60.9) (width 0.2) (layer "F.Cu") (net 4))
 (via (at 196.57 60.905) (size 0.6) (drill 0.3) (layers "F.Cu" "B.Cu") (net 4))
 (segment (start 166.28 70.42) (end 180.043 56.657) (width 0.2) (layer "B.Cu") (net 4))
 (segment (start 180.043 56.657) (end 193.157 56.657) (width 0.2) (layer "B.Cu") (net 4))
 (segment (start 193.157 56.657) (end 197.1 60.6) (width 0.2) (layer "B.Cu") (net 4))
 (segment (start 197.1 60.6) (end 196.8 60.9) (width 0.2) (layer "B.Cu") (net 4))
 (segment (start 190.572 56.657) (end 193.07 59.155) (width 0.2) (layer "F.Cu") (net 3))
 (segment (start 159.708 56.657) (end 190.572 56.657) (width 0.2) (layer "F.Cu") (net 3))
 (segment (start 155.41 60.955) (end 159.708 56.657) (width 0.2) (layer "F.Cu") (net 3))
 (segment (start 184.3 68.12) (end 181.52 65.34) (width 0.2) (layer "B.Cu") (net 14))
 (segment (start 184.3 86) (end 181.91025 88.38975) (width 0.2) (layer "B.Cu") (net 14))
 (segment (start 184.3 86) (end 184.3 68.12) (width 0.2) (layer "B.Cu") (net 14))
 (segment (start 181.91025 88.38975) (end 175.375816 88.38975) (width 0.2) (layer "B.Cu") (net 14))
 (segment (start 175.375816 88.38975) (end 174.933566 87.9475) (width 0.2) (layer "B.Cu") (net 14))
 (segment (start 174.933566 87.9475) (end 170.33875 87.9475) (width 0.2) (layer "B.Cu") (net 14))
 (segment (start 153.698 76.327274) (end 164.685274 65.34) (width 0.2) (layer "F.Cu") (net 12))
 (segment (start 159.915936 139.35475) (end 159.09525 138.534064) (width 0.2) (layer "F.Cu") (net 12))
 (segment (start 153.698 140.3322) (end 153.698 76.327274) (width 0.2) (layer "F.Cu") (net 12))
 (segment (start 160.49625 135.972436) (end 161.89725 137.373436) (width 0.2) (layer "F.Cu") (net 12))
 (segment (start 159.09525 138.534064) (end 156.668314 140.961) (width 0.2) (layer "F.Cu") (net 12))
 (segment (start 161.89725 137.373436) (end 161.89725 138.534064) (width 0.2) (layer "F.Cu") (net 12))
 (segment (start 161.89725 138.534064) (end 161.076564 139.35475) (width 0.2) (layer "F.Cu") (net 12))
 (segment (start 156.668314 140.961) (end 154.3268 140.961) (width 0.2) (layer "F.Cu") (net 12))
 (segment (start 164.685274 65.34) (end 166.28 65.34) (width 0.2) (layer "F.Cu") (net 12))
 (segment (start 154.3268 140.961) (end 153.698 140.3322) (width 0.2) (layer "F.Cu") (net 12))
 (segment (start 160.49625 111.76) (end 160.49625 135.972436) (width 0.2) (layer "F.Cu") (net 12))
 (segment (start 161.076564 139.35475) (end 159.915936 139.35475) (width 0.2) (layer "F.Cu") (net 12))
 (segment (start 154.099 76.493374) (end 154.099 140.1661) (width 0.2) (layer "F.Cu") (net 2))
 (segment (start 157.24625 137.95375) (end 160.49625 137.95375) (width 0.2) (layer "F.Cu") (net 2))
 (segment (start 173.87369 66.403) (end 164.189374 66.403) (width 0.2) (layer "F.Cu") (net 2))
 (segment (start 181.07969 59.197) (end 173.87369 66.403) (width 0.2) (layer "F.Cu") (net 2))
 (segment (start 164.189374 66.403) (end 154.099 76.493374) (width 0.2) (layer "F.Cu") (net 2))
 (segment (start 183.872 61.061626) (end 183.872 59.458374) (width 0.2) (layer "F.Cu") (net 2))
 (segment (start 154.64 140.56) (end 157.24625 137.95375) (width 0.2) (layer "F.Cu") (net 2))
 (segment (start 154.4929 140.56) (end 154.64 140.56) (width 0.2) (layer "F.Cu") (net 2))
 (segment (start 154.099 140.1661) (end 154.4929 140.56) (width 0.2) (layer "F.Cu") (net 2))
 (segment (start 181.52 62.8) (end 182.133626 62.8) (width 0.2) (layer "F.Cu") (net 2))
 (segment (start 182.133626 62.8) (end 183.872 61.061626) (width 0.2) (layer "F.Cu") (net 2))
 (segment (start 183.610626 59.197) (end 181.07969 59.197) (width 0.2) (layer "F.Cu") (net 2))
 (segment (start 183.872 59.458374) (end 183.610626 59.197) (width 0.2) (layer "F.Cu") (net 2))
 (segment (start 166.265936 110.621) (end 161.849 106.204064) (width 0.2) (layer "F.Cu") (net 7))
 (segment (start 161.849 106.204064) (end 161.849 90.091) (width 0.2) (layer "F.Cu") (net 7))
 (segment (start 175.075 116.8) (end 173.605564 116.8) (width 0.2) (layer "F.Cu") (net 7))
 (segment (start 181.52 70.42) (end 161.849 90.091) (width 0.2) (layer "F.Cu") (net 7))
 (segment (start 167.426564 110.621) (end 166.265936 110.621) (width 0.2) (layer "F.Cu") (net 7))
 (segment (start 173.605564 116.8) (end 167.426564 110.621) (width 0.2) (layer "F.Cu") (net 7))
 (segment (start 181.472 105.503) (end 175.175 111.8) (width 0.2) (layer "F.Cu") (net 6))
 (segment (start 182.133626 67.88) (end 183.872 69.618374) (width 0.2) (layer "F.Cu") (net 6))
 (segment (start 181.52 67.88) (end 182.133626 67.88) (width 0.2) (layer "F.Cu") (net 6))
 (segment (start 175.6 111.8) (end 175.5401 111.8) (width 0.2) (layer "F.Cu") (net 6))
 (segment (start 183.872 105.503) (end 181.472 105.503) (width 0.2) (layer "F.Cu") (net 6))
 (segment (start 175.5401 111.8) (end 175.35755 111.98255) (width 0.2) (layer "F.Cu") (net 6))
 (segment (start 183.872 69.618374) (end 183.872 105.503) (width 0.2) (layer "F.Cu") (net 6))
 (segment (start 167.343 66.817) (end 166.28 67.88) (width 0.2) (layer "F.Cu") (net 13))
 (segment (start 183.610626 66.817) (end 167.343 66.817) (width 0.2) (layer "F.Cu") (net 13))
 (segment (start 166.28 67.88) (end 165.20237 67.88) (width 0.2) (layer "F.Cu") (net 13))
 (segment (start 179.6 137.95375) (end 185.391314 137.95375) (width 0.2) (layer "F.Cu") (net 13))
 (segment (start 187.351 70.557374) (end 183.610626 66.817) (width 0.2) (layer "F.Cu") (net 13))
 (segment (start 187.351 135.994064) (end 187.351 70.557374) (width 0.2) (layer "F.Cu") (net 13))
 (segment (start 185.391314 137.95375) (end 187.351 135.994064) (width 0.2) (layer "F.Cu") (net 13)))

